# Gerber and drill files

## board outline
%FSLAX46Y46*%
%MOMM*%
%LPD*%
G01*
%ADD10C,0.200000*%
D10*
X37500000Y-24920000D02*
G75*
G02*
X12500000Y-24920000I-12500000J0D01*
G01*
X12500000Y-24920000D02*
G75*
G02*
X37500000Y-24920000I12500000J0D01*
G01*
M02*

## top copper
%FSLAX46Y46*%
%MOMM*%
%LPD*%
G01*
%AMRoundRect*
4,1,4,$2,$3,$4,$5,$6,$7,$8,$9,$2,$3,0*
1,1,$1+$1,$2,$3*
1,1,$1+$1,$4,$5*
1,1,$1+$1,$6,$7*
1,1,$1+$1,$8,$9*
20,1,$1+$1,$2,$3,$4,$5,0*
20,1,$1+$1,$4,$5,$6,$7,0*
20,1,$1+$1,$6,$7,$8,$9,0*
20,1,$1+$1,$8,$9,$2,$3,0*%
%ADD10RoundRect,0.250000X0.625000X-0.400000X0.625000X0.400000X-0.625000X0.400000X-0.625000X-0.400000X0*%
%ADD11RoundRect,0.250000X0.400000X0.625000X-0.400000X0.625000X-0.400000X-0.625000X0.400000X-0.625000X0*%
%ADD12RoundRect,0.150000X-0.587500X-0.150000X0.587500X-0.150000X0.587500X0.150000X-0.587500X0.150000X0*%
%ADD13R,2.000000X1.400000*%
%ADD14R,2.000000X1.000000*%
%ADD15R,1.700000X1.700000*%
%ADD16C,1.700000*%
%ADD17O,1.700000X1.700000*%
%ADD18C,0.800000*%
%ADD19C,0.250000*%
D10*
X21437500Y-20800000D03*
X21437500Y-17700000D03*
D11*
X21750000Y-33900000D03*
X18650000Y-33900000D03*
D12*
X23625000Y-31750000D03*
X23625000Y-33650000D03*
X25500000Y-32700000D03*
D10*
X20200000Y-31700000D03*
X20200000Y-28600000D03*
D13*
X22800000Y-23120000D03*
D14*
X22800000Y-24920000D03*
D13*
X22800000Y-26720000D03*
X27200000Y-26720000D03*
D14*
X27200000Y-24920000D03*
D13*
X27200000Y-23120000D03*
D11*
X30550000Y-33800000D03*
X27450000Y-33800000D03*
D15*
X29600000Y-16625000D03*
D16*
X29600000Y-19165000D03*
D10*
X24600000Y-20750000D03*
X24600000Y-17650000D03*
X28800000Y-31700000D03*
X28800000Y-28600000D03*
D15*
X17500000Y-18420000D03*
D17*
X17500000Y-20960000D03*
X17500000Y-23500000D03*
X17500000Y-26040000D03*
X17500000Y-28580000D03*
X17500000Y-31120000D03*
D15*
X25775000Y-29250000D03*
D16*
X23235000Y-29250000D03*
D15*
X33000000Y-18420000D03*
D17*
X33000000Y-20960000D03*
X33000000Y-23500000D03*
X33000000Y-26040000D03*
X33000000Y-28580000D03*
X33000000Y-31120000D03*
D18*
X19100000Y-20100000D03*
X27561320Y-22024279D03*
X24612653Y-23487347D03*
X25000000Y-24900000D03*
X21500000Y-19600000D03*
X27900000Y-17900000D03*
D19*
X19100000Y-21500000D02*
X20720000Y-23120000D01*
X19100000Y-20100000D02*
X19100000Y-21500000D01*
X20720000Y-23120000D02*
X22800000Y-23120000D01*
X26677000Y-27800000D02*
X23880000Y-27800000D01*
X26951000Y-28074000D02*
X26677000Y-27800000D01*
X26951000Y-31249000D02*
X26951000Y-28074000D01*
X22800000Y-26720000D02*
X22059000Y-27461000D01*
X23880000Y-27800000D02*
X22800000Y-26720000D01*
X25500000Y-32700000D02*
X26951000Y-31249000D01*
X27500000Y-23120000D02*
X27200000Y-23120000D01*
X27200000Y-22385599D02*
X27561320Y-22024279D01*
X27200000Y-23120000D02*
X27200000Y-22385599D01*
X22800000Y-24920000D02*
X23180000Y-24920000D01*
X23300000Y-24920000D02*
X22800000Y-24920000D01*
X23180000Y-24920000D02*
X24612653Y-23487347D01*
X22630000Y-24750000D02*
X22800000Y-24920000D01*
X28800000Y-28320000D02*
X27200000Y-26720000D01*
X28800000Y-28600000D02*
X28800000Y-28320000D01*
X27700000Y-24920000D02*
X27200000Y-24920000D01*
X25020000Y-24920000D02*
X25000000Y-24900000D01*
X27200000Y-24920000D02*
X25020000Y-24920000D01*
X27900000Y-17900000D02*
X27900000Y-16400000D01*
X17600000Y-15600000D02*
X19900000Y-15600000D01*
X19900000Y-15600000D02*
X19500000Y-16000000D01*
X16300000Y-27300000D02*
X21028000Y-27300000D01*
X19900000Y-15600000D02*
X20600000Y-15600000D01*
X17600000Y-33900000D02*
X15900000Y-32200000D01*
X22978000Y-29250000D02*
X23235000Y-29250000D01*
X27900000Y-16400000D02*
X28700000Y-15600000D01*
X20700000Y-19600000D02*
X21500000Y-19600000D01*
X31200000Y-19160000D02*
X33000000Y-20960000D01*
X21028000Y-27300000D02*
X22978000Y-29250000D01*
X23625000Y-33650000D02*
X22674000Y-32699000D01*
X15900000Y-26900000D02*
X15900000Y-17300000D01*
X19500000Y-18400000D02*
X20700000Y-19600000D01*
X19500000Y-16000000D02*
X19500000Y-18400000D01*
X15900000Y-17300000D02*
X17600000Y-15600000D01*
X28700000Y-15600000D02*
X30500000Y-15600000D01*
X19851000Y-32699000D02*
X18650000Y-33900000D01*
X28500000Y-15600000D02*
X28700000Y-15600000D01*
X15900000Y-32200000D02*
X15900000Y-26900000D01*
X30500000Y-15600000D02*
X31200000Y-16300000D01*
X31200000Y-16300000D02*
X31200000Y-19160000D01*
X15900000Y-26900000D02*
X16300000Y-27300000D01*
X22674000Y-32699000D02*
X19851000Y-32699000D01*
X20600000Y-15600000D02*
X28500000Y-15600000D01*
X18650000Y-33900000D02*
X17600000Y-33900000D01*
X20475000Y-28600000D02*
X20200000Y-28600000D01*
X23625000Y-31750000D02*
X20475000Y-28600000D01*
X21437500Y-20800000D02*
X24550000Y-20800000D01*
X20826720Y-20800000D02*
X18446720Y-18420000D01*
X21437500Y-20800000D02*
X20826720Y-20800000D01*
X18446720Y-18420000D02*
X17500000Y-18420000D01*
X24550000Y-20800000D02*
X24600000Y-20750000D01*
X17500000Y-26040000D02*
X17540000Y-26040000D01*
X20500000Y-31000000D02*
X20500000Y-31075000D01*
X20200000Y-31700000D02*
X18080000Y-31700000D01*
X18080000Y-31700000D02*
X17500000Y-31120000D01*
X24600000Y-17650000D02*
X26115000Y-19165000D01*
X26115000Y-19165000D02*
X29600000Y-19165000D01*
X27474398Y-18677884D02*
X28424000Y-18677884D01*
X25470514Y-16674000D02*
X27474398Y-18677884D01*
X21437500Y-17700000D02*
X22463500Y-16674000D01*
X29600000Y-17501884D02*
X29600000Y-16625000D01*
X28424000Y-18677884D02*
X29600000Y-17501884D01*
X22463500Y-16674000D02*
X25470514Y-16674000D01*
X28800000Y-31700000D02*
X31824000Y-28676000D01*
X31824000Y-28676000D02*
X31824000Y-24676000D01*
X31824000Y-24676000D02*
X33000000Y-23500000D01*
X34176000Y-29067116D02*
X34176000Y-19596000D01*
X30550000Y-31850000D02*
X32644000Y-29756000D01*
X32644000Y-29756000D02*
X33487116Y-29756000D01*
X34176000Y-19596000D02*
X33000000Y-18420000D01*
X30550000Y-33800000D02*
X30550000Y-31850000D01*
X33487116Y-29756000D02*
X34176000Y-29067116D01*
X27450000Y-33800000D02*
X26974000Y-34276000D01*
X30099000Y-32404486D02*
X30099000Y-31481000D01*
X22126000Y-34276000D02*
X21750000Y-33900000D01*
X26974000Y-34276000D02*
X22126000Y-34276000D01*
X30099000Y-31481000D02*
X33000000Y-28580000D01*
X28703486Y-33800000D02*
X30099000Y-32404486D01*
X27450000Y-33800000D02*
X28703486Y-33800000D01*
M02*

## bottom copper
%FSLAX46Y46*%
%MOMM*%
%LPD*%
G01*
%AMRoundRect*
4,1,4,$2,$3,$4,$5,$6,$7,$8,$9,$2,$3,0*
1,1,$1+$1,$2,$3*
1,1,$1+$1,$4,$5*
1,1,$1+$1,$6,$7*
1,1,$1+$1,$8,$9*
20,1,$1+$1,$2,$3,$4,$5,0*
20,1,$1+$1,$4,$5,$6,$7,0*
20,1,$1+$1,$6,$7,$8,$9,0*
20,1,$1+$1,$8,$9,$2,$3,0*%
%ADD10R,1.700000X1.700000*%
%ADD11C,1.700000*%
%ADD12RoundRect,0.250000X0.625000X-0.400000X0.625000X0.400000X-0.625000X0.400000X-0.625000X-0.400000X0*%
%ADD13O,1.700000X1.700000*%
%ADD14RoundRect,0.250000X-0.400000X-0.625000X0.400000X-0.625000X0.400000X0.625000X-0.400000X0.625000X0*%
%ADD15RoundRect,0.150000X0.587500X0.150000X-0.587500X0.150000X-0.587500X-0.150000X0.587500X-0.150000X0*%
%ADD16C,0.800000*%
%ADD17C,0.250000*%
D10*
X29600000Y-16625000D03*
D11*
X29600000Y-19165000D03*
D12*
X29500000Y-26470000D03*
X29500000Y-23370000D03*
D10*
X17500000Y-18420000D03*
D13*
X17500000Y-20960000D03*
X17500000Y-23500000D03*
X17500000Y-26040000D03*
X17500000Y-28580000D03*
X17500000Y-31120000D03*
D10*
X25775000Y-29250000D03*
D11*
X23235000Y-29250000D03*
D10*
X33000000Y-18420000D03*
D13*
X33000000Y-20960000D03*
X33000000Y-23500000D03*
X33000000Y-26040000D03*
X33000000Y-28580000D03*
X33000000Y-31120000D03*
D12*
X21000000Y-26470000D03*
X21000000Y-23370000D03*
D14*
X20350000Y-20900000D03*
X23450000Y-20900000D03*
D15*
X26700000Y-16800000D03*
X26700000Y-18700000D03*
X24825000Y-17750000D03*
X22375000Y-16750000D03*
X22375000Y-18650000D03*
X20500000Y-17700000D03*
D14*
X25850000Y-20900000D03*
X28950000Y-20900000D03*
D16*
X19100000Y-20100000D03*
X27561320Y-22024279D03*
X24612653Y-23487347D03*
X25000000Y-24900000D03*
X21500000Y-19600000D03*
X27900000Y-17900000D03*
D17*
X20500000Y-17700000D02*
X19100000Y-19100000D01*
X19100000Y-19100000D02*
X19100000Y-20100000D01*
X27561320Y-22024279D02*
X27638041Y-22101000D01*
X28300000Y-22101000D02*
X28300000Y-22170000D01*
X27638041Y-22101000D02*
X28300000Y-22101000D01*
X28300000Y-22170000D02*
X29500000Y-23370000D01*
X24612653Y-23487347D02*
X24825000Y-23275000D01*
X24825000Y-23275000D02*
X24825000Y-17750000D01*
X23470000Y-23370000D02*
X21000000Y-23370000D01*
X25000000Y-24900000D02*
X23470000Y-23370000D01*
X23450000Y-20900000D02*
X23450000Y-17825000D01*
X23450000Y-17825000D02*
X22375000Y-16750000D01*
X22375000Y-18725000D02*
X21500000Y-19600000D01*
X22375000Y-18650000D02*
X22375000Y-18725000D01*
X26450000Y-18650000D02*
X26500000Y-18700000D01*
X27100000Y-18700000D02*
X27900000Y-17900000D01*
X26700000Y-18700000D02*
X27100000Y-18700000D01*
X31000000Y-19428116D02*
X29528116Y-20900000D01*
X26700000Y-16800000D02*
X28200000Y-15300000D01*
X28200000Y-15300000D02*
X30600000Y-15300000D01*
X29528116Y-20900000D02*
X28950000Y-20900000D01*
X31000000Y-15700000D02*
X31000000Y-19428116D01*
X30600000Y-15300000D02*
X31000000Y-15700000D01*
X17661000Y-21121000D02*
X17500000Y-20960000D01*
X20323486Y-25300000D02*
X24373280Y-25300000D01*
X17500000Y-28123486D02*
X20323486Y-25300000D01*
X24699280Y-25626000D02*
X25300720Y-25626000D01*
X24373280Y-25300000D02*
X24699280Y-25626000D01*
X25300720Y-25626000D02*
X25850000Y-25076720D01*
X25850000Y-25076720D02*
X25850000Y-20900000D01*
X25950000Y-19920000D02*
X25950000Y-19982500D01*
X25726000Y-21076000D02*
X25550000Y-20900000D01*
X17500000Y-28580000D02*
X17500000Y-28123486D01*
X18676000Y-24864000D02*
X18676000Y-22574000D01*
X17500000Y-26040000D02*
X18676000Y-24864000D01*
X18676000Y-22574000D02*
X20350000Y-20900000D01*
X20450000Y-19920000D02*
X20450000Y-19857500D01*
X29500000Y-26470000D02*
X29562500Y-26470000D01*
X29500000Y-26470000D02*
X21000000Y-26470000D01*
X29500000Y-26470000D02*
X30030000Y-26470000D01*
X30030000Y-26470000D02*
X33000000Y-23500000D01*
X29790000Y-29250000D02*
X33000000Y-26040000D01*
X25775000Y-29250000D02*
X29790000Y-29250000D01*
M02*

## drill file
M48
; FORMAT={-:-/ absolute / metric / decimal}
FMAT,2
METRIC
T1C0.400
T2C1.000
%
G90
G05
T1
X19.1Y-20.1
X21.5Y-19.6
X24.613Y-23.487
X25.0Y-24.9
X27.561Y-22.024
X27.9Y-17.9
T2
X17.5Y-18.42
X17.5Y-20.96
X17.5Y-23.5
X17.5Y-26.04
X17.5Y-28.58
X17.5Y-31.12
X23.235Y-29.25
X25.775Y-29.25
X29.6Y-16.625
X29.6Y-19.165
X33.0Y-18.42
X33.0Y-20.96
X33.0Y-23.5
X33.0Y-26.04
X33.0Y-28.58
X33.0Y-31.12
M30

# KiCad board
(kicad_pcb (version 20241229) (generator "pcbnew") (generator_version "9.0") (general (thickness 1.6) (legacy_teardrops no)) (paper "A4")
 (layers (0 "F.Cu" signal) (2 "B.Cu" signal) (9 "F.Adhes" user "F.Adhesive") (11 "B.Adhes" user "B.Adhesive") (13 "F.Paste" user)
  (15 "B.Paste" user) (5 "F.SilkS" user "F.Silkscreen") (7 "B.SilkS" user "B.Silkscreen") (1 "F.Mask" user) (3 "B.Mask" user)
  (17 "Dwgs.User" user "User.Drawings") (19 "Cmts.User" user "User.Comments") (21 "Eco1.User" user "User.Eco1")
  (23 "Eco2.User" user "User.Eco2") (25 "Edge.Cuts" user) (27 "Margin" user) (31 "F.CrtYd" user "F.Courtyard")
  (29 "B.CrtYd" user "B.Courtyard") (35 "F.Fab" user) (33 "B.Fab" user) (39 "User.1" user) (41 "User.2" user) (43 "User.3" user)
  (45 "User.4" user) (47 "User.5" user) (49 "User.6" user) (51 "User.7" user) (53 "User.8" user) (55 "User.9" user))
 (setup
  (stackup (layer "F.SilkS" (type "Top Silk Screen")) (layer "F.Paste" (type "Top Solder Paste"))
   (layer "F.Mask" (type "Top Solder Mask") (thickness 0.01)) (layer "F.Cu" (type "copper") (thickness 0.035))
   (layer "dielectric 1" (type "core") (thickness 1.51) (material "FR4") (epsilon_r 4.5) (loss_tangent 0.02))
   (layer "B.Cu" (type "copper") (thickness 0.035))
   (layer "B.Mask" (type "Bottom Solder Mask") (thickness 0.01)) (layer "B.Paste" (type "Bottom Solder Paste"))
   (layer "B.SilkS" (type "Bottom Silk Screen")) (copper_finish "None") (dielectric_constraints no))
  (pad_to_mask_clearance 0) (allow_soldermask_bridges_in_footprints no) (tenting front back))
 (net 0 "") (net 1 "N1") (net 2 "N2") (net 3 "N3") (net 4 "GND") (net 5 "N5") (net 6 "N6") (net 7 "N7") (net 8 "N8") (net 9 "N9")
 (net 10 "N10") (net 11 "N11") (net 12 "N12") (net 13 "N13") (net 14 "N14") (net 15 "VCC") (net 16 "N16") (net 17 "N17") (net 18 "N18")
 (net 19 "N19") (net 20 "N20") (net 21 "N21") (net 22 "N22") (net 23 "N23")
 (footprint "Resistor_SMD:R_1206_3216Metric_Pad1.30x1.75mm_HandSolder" (layer "F.Cu") (at 21.4375 19.25 90)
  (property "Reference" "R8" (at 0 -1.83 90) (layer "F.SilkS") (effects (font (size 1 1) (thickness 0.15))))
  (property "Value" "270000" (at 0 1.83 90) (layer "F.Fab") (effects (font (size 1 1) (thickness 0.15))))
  (pad "1" smd roundrect (at -1.55 0 90) (size 1.3 1.75) (layers "F.Cu" "F.Mask" "F.Paste") (roundrect_rratio 0.192308) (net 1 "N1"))
  (pad "2" smd roundrect (at 1.55 0 90) (size 1.3 1.75) (layers "F.Cu" "F.Mask" "F.Paste") (roundrect_rratio 0.192308) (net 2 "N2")))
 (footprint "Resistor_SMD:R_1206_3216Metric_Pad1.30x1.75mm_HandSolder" (layer "F.Cu") (at 20.2 33.9 180)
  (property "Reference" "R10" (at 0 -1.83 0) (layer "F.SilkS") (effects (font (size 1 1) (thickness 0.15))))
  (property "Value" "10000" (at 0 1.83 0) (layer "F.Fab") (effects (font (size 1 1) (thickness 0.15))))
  (pad "1" smd roundrect (at -1.55 0 180) (size 1.3 1.75) (layers "F.Cu" "F.Mask" "F.Paste") (roundrect_rratio 0.192308) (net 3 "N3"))
  (pad "2" smd roundrect (at 1.55 0 180) (size 1.3 1.75) (layers "F.Cu" "F.Mask" "F.Paste") (roundrect_rratio 0.192308) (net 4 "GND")))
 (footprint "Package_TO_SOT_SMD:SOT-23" (layer "F.Cu") (at 24.5625 32.7)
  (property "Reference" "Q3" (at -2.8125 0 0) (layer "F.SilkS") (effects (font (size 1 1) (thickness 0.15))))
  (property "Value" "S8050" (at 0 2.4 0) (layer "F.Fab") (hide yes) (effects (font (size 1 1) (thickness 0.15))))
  (pad "1" smd roundrect (at -0.9375 -0.95) (size 1.475 0.6) (layers "F.Cu" "F.Mask" "F.Paste") (roundrect_rratio 0.25) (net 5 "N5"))
  (pad "2" smd roundrect (at -0.9375 0.95) (size 1.475 0.6) (layers "F.Cu" "F.Mask" "F.Paste") (roundrect_rratio 0.25) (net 4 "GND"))
  (pad "3" smd roundrect (at 0.9375 0) (size 1.475 0.6) (layers "F.Cu" "F.Mask" "F.Paste") (roundrect_rratio 0.25) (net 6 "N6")))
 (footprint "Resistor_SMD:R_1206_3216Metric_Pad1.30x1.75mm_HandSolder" (layer "F.Cu") (at 20.2 30.15 90)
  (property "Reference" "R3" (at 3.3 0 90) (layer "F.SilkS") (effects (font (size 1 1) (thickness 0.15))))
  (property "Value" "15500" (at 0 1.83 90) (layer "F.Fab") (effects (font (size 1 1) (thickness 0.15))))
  (pad "1" smd roundrect (at -1.55 0 90) (size 1.3 1.75) (layers "F.Cu" "F.Mask" "F.Paste") (roundrect_rratio 0.192308) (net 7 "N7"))
  (pad "2" smd roundrect (at 1.55 0 90) (size 1.3 1.75) (layers "F.Cu" "F.Mask" "F.Paste") (roundrect_rratio 0.192308) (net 5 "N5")))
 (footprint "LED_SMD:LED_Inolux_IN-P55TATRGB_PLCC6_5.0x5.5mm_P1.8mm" (layer "F.Cu") (at 25 24.92)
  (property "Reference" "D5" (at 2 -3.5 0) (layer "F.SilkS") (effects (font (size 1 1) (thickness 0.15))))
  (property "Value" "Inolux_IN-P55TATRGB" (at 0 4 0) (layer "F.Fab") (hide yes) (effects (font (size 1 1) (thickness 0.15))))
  (pad "1" smd rect (at -2.2 -1.8) (size 2 1.4) (layers "F.Cu" "F.Mask" "F.Paste") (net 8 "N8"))
  (pad "2" smd rect (at -2.2 0) (size 2 1) (layers "F.Cu" "F.Mask" "F.Paste") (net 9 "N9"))
  (pad "3" smd rect (at -2.2 1.8) (size 2 1.4) (layers "F.Cu" "F.Mask" "F.Paste") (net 6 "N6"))
  (pad "4" smd rect (at 2.2 1.8) (size 2 1.4) (layers "F.Cu" "F.Mask" "F.Paste") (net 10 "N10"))
  (pad "5" smd rect (at 2.2 0) (size 2 1) (layers "F.Cu" "F.Mask" "F.Paste") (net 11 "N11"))
  (pad "6" smd rect (at 2.2 -1.8) (size 2 1.4) (layers "F.Cu" "F.Mask" "F.Paste") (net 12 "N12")))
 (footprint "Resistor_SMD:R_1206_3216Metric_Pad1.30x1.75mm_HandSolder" (layer "F.Cu") (at 29 33.8 180)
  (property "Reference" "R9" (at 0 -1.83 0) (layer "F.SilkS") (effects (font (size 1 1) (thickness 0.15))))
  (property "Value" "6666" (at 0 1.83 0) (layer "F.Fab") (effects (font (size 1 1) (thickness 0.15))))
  (pad "1" smd roundrect (at -1.55 0 180) (size 1.3 1.75) (layers "F.Cu" "F.Mask" "F.Paste") (roundrect_rratio 0.192308) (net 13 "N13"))
  (pad "2" smd roundrect (at 1.55 0 180) (size 1.3 1.75) (layers "F.Cu" "F.Mask" "F.Paste") (roundrect_rratio 0.192308) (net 3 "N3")))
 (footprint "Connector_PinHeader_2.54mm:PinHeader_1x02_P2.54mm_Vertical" (layer "F.Cu") (at 29.6 16.625)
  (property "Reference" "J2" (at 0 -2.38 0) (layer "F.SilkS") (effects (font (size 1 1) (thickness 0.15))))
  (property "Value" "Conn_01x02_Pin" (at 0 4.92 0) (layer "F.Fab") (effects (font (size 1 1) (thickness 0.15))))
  (pad "1" thru_hole rect (at 0 0) (size 1.7 1.7) (drill 1) (layers "*.Cu" "*.Mask") (remove_unused_layers no) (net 2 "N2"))
  (pad "2" thru_hole circle (at 0 2.54) (size 1.7 1.7) (drill 1) (layers "*.Cu" "*.Mask") (remove_unused_layers no) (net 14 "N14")))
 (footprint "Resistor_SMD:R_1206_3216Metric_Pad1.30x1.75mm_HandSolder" (layer "F.Cu") (at 24.6 19.2 90)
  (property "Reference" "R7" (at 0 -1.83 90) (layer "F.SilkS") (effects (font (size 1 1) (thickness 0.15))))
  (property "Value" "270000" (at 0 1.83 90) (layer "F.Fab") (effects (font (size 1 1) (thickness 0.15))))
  (pad "1" smd roundrect (at -1.55 0 90) (size 1.3 1.75) (layers "F.Cu" "F.Mask" "F.Paste") (roundrect_rratio 0.192308) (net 1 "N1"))
  (pad "2" smd roundrect (at 1.55 0 90) (size 1.3 1.75) (layers "F.Cu" "F.Mask" "F.Paste") (roundrect_rratio 0.192308) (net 14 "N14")))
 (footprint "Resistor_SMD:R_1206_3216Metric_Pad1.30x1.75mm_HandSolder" (layer "F.Cu") (at 28.8 30.15 90)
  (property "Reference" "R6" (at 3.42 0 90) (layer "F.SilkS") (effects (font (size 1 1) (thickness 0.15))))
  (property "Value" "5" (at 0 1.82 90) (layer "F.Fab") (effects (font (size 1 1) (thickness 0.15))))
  (pad "1" smd roundrect (at -1.55 0 90) (size 1.3 1.75) (layers "F.Cu" "F.Mask" "F.Paste") (roundrect_rratio 0.192308) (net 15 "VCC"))
  (pad "2" smd roundrect (at 1.55 0 90) (size 1.3 1.75) (layers "F.Cu" "F.Mask" "F.Paste") (roundrect_rratio 0.192308) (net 10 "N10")))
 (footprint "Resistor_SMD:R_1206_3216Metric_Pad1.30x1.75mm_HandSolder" (layer "B.Cu") (at 29.5 24.92 90)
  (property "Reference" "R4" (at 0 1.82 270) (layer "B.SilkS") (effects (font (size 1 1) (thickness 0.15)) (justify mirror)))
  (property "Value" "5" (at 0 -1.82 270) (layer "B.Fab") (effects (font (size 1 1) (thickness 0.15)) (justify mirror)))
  (pad "1" smd roundrect (at -1.55 0 90) (size 1.3 1.75) (layers "B.Cu" "B.Mask" "B.Paste") (roundrect_rratio 0.192308) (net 15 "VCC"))
  (pad "2" smd roundrect (at 1.55 0 90) (size 1.3 1.75) (layers "B.Cu" "B.Mask" "B.Paste") (roundrect_rratio 0.192308) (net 12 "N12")))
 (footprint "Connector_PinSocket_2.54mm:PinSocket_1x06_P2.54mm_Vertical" (layer "B.Cu") (at 17.5 18.42 180)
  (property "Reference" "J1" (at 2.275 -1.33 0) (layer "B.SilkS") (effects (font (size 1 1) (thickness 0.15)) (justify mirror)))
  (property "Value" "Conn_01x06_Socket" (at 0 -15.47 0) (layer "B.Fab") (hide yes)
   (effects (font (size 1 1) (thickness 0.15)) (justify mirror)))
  (pad "1" thru_hole rect (at 0 0 180) (size 1.7 1.7) (drill 1) (layers "*.Cu" "*.Mask") (remove_unused_layers no) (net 1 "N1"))
  (pad "2" thru_hole oval (at 0 -2.54 180) (size 1.7 1.7) (drill 1) (layers "*.Cu" "*.Mask") (remove_unused_layers no) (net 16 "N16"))
  (pad "3" thru_hole oval (at 0 -5.08 180) (size 1.7 1.7) (drill 1) (layers "*.Cu" "*.Mask") (remove_unused_layers no) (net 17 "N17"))
  (pad "4" thru_hole oval (at 0 -7.62 180) (size 1.7 1.7) (drill 1) (layers "*.Cu" "*.Mask") (remove_unused_layers no) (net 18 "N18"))
  (pad "5" thru_hole oval (at 0 -10.16 180) (size 1.7 1.7) (drill 1) (layers "*.Cu" "*.Mask") (remove_unused_layers no) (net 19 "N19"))
  (pad "6" thru_hole oval (at 0 -12.7 180) (size 1.7 1.7) (drill 1) (layers "*.Cu" "*.Mask") (remove_unused_layers no) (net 7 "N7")))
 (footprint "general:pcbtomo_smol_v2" (layer "B.Cu") (at 24.275 29.5 180)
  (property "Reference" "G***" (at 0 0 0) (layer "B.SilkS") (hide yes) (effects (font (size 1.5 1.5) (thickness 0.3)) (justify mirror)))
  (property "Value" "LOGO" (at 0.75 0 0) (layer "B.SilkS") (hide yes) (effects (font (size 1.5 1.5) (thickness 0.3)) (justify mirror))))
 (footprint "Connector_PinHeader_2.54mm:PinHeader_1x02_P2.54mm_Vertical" (layer "B.Cu") (at 25.775 29.25 90)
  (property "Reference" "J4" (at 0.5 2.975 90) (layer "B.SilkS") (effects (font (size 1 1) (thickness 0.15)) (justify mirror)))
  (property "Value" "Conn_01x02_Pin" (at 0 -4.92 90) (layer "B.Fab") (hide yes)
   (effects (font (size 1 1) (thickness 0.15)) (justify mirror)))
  (pad "1" thru_hole rect (at 0 0 90) (size 1.7 1.7) (drill 1) (layers "*.Cu" "*.Mask") (remove_unused_layers no) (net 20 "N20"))
  (pad "2" thru_hole circle (at 0 -2.54 90) (size 1.7 1.7) (drill 1) (layers "*.Cu" "*.Mask") (remove_unused_layers no) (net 4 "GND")))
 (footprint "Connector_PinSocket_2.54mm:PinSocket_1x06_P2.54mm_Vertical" (layer "B.Cu") (at 33 18.42 180)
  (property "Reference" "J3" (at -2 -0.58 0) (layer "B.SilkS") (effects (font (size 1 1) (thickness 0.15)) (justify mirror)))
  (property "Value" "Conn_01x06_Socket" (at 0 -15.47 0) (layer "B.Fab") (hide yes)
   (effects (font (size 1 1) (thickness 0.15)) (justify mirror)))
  (pad "1" thru_hole rect (at 0 0 180) (size 1.7 1.7) (drill 1) (layers "*.Cu" "*.Mask") (remove_unused_layers no) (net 13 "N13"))
  (pad "2" thru_hole oval (at 0 -2.54 180) (size 1.7 1.7) (drill 1) (layers "*.Cu" "*.Mask") (remove_unused_layers no) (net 4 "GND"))
  (pad "3" thru_hole oval (at 0 -5.08 180) (size 1.7 1.7) (drill 1) (layers "*.Cu" "*.Mask") (remove_unused_layers no) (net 15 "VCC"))
  (pad "4" thru_hole oval (at 0 -7.62 180) (size 1.7 1.7) (drill 1) (layers "*.Cu" "*.Mask") (remove_unused_layers no) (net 20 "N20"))
  (pad "5" thru_hole oval (at 0 -10.16 180) (size 1.7 1.7) (drill 1) (layers "*.Cu" "*.Mask") (remove_unused_layers no) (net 3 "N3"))
  (pad "6" thru_hole oval (at 0 -12.7 180) (size 1.7 1.7) (drill 1) (layers "*.Cu" "*.Mask") (remove_unused_layers no) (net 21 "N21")))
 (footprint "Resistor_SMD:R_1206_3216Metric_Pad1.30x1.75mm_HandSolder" (layer "B.Cu") (at 21 24.92 90)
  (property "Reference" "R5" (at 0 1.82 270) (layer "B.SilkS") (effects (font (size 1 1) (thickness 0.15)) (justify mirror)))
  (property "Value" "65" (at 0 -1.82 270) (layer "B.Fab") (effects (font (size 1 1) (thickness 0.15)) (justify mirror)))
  (pad "1" smd roundrect (at -1.55 0 90) (size 1.3 1.75) (layers "B.Cu" "B.Mask" "B.Paste") (roundrect_rratio 0.192308) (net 15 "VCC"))
  (pad "2" smd roundrect (at 1.55 0 90) (size 1.3 1.75) (layers "B.Cu" "B.Mask" "B.Paste") (roundrect_rratio 0.192308) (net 11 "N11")))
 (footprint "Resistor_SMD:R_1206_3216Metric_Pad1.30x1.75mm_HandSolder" (layer "B.Cu") (at 21.9 20.9)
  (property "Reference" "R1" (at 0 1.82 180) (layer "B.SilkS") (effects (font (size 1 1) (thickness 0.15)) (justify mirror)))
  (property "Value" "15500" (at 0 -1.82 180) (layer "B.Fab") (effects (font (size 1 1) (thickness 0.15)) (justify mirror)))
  (pad "1" smd roundrect (at -1.55 0) (size 1.3 1.75) (layers "B.Cu" "B.Mask" "B.Paste") (roundrect_rratio 0.192308) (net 18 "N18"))
  (pad "2" smd roundrect (at 1.55 0) (size 1.3 1.75) (layers "B.Cu" "B.Mask" "B.Paste") (roundrect_rratio 0.192308) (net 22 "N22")))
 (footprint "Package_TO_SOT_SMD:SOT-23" (layer "B.Cu") (at 25.7625 17.75 180)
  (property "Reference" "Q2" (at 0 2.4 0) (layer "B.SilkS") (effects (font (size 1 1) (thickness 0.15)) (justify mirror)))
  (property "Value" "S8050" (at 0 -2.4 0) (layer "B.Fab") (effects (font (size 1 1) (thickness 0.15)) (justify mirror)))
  (pad "1" smd roundrect (at -0.9375 0.95 180) (size 1.475 0.6) (layers "B.Cu" "B.Mask" "B.Paste") (roundrect_rratio 0.25) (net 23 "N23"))
  (pad "2" smd roundrect (at -0.9375 -0.95 180) (size 1.475 0.6) (layers "B.Cu" "B.Mask" "B.Paste") (roundrect_rratio 0.25) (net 4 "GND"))
  (pad "3" smd roundrect (at 0.9375 0 180) (size 1.475 0.6) (layers "B.Cu" "B.Mask" "B.Paste") (roundrect_rratio 0.25) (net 9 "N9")))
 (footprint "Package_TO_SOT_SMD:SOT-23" (layer "B.Cu") (at 21.4375 17.7 180)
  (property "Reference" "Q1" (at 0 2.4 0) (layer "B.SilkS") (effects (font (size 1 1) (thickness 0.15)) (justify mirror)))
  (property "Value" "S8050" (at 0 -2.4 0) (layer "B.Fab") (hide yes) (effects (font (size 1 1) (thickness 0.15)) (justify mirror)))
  (pad "1" smd roundrect (at -0.9375 0.95 180) (size 1.475 0.6) (layers "B.Cu" "B.Mask" "B.Paste") (roundrect_rratio 0.25) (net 22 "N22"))
  (pad "2" smd roundrect (at -0.9375 -0.95 180) (size 1.475 0.6) (layers "B.Cu" "B.Mask" "B.Paste") (roundrect_rratio 0.25) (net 4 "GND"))
  (pad "3" smd roundrect (at 0.9375 0 180) (size 1.475 0.6) (layers "B.Cu" "B.Mask" "B.Paste") (roundrect_rratio 0.25) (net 8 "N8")))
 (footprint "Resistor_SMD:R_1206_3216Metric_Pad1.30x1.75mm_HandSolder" (layer "B.Cu") (at 27.4 20.9)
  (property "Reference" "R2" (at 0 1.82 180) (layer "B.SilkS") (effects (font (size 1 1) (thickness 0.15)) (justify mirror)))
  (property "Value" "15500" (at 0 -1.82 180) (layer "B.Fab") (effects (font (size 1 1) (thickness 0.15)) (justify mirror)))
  (pad "1" smd roundrect (at -1.55 0) (size 1.3 1.75) (layers "B.Cu" "B.Mask" "B.Paste") (roundrect_rratio 0.192308) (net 19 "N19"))
  (pad "2" smd roundrect (at 1.55 0) (size 1.3 1.75) (layers "B.Cu" "B.Mask" "B.Paste") (roundrect_rratio 0.192308) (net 23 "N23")))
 (gr_circle (center 25 24.92) (end 37.5 24.92) (stroke (width 0.2) (type default)) (fill no) (layer "Edge.Cuts"))
 (segment (start 19.1 21.5) (end 20.72 23.12) (width 0.25) (layer "F.Cu") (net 8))
 (segment (start 19.1 20.1) (end 19.1 21.5) (width 0.25) (layer "F.Cu") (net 8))
 (segment (start 20.72 23.12) (end 22.8 23.12) (width 0.25) (layer "F.Cu") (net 8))
 (via (at 19.1 20.1) (size 0.8) (drill 0.4) (layers "F.Cu" "B.Cu") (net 8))
 (segment (start 20.5 17.7) (end 19.1 19.1) (width 0.25) (layer "B.Cu") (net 8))
 (segment (start 19.1 19.1) (end 19.1 20.1) (width 0.25) (layer "B.Cu") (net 8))
 (segment (start 26.677 27.8) (end 23.88 27.8) (width 0.25) (layer "F.Cu") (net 6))
 (segment (start 26.951 28.074) (end 26.677 27.8) (width 0.25) (layer "F.Cu") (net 6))
 (segment (start 26.951 31.249) (end 26.951 28.074) (width 0.25) (layer "F.Cu") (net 6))
 (segment (start 22.8 26.72) (end 22.059 27.461) (width 0.25) (layer "F.Cu") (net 6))
 (segment (start 23.88 27.8) (end 22.8 26.72) (width 0.25) (layer "F.Cu") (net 6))
 (segment (start 25.5 32.7) (end 26.951 31.249) (width 0.25) (layer "F.Cu") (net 6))
 (segment (start 27.5 23.12) (end 27.2 23.12) (width 0.25) (layer "F.Cu") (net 12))
 (segment (start 27.2 22.385599) (end 27.56132 22.024279) (width 0.25) (layer "F.Cu") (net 12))
 (segment (start 27.2 23.12) (end 27.2 22.385599) (width 0.25) (layer "F.Cu") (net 12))
 (via (at 27.56132 22.024279) (size 0.8) (drill 0.4) (layers "F.Cu" "B.Cu") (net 12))
 (segment (start 27.56132 22.024279) (end 27.638041 22.101) (width 0.25) (layer "B.Cu") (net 12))
 (segment (start 28.3 22.101) (end 28.3 22.17) (width 0.25) (layer "B.Cu") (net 12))
 (segment (start 27.638041 22.101) (end 28.3 22.101) (width 0.25) (layer "B.Cu") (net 12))
 (segment (start 28.3 22.17) (end 29.5 23.37) (width 0.25) (layer "B.Cu") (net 12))
 (segment (start 22.8 24.92) (end 23.18 24.92) (width 0.25) (layer "F.Cu") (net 9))
 (segment (start 23.3 24.92) (end 22.8 24.92) (width 0.25) (layer "F.Cu") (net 9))
 (segment (start 23.18 24.92) (end 24.612653 23.487347) (width 0.25) (layer "F.Cu") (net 9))
 (segment (start 22.63 24.75) (end 22.8 24.92) (width 0.25) (layer "F.Cu") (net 9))
 (via (at 24.612653 23.487347) (size 0.8) (drill 0.4) (layers "F.Cu" "B.Cu") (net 9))
 (segment (start 24.612653 23.487347) (end 24.825 23.275) (width 0.25) (layer "B.Cu") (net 9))
 (segment (start 24.825 23.275) (end 24.825 17.75) (width 0.25) (layer "B.Cu") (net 9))
 (segment (start 28.8 28.32) (end 27.2 26.72) (width 0.25) (layer "F.Cu") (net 10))
 (segment (start 28.8 28.6) (end 28.8 28.32) (width 0.25) (layer "F.Cu") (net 10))
 (segment (start 27.7 24.92) (end 27.2 24.92) (width 0.25) (layer "F.Cu") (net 11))
 (segment (start 25.02 24.92) (end 25 24.9) (width 0.25) (layer "F.Cu") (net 11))
 (segment (start 27.2 24.92) (end 25.02 24.92) (width 0.25) (layer "F.Cu") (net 11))
 (via (at 25 24.9) (size 0.8) (drill 0.4) (layers "F.Cu" "B.Cu") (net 11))
 (segment (start 23.47 23.37) (end 21 23.37) (width 0.25) (layer "B.Cu") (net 11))
 (segment (start 25 24.9) (end 23.47 23.37) (width 0.25) (layer "B.Cu") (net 11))
 (segment (start 23.45 20.9) (end 23.45 17.825) (width 0.25) (layer "B.Cu") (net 22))
 (segment (start 23.45 17.825) (end 22.375 16.75) (width 0.25) (layer "B.Cu") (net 22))
 (segment (start 27.9 17.9) (end 27.9 16.4) (width 0.25) (layer "F.Cu") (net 4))
 (segment (start 17.6 15.6) (end 19.9 15.6) (width 0.25) (layer "F.Cu") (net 4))
 (segment (start 19.9 15.6) (end 19.5 16) (width 0.25) (layer "F.Cu") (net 4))
 (segment (start 16.3 27.3) (end 21.028 27.3) (width 0.25) (layer "F.Cu") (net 4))
 (segment (start 19.9 15.6) (end 20.6 15.6) (width 0.25) (layer "F.Cu") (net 4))
 (segment (start 17.6 33.9) (end 15.9 32.2) (width 0.25) (layer "F.Cu") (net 4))
 (segment (start 22.978 29.25) (end 23.235 29.25) (width 0.25) (layer "F.Cu") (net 4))
 (segment (start 27.9 16.4) (end 28.7 15.6) (width 0.25) (layer "F.Cu") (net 4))
 (segment (start 20.7 19.6) (end 21.5 19.6) (width 0.25) (layer "F.Cu") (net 4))
 (segment (start 31.2 19.16) (end 33 20.96) (width 0.25) (layer "F.Cu") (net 4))
 (segment (start 21.028 27.3) (end 22.978 29.25) (width 0.25) (layer "F.Cu") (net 4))
 (segment (start 23.625 33.65) (end 22.674 32.699) (width 0.25) (layer "F.Cu") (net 4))
 (segment (start 15.9 26.9) (end 15.9 17.3) (width 0.25) (layer "F.Cu") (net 4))
 (segment (start 19.5 18.4) (end 20.7 19.6) (width 0.25) (layer "F.Cu") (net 4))
 (segment (start 19.5 16) (end 19.5 18.4) (width 0.25) (layer "F.Cu") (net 4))
 (segment (start 15.9 17.3) (end 17.6 15.6) (width 0.25) (layer "F.Cu") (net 4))
 (segment (start 28.7 15.6) (end 30.5 15.6) (width 0.25) (layer "F.Cu") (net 4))
 (segment (start 19.851 32.699) (end 18.65 33.9) (width 0.25) (layer "F.Cu") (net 4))
 (segment (start 28.5 15.6) (end 28.7 15.6) (width 0.25) (layer "F.Cu") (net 4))
 (segment (start 15.9 32.2) (end 15.9 26.9) (width 0.25) (layer "F.Cu") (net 4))
 (segment (start 30.5 15.6) (end 31.2 16.3) (width 0.25) (layer "F.Cu") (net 4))
 (segment (start 31.2 16.3) (end 31.2 19.16) (width 0.25) (layer "F.Cu") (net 4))
 (segment (start 15.9 26.9) (end 16.3 27.3) (width 0.25) (layer "F.Cu") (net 4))
 (segment (start 22.674 32.699) (end 19.851 32.699) (width 0.25) (layer "F.Cu") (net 4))
 (segment (start 20.6 15.6) (end 28.5 15.6) (width 0.25) (layer "F.Cu") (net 4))
 (segment (start 18.65 33.9) (end 17.6 33.9) (width 0.25) (layer "F.Cu") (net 4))
 (via (at 21.5 19.6) (size 0.8) (drill 0.4) (layers "F.Cu" "B.Cu") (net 4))
 (via (at 27.9 17.9) (size 0.8) (drill 0.4) (layers "F.Cu" "B.Cu") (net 4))
 (segment (start 22.375 18.725) (end 21.5 19.6) (width 0.25) (layer "B.Cu") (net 4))
 (segment (start 22.375 18.65) (end 22.375 18.725) (width 0.25) (layer "B.Cu") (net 4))
 (segment (start 26.45 18.65) (end 26.5 18.7) (width 0.25) (layer "B.Cu") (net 4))
 (segment (start 27.1 18.7) (end 27.9 17.9) (width 0.25) (layer "B.Cu") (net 4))
 (segment (start 26.7 18.7) (end 27.1 18.7) (width 0.25) (layer "B.Cu") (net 4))
 (segment (start 31 19.428116) (end 29.528116 20.9) (width 0.25) (layer "B.Cu") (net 23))
 (segment (start 26.7 16.8) (end 28.2 15.3) (width 0.25) (layer "B.Cu") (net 23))
 (segment (start 28.2 15.3) (end 30.6 15.3) (width 0.25) (layer "B.Cu") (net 23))
 (segment (start 29.528116 20.9) (end 28.95 20.9) (width 0.25) (layer "B.Cu") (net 23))
 (segment (start 31 15.7) (end 31 19.428116) (width 0.25) (layer "B.Cu") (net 23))
 (segment (start 30.6 15.3) (end 31 15.7) (width 0.25) (layer "B.Cu") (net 23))
 (segment (start 20.475 28.6) (end 20.2 28.6) (width 0.25) (layer "F.Cu") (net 5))
 (segment (start 23.625 31.75) (end 20.475 28.6) (width 0.25) (layer "F.Cu") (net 5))
 (segment (start 17.661 21.121) (end 17.5 20.96) (width 0.25) (layer "B.Cu") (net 16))
 (segment (start 20.323486 25.3) (end 24.37328 25.3) (width 0.25) (layer "B.Cu") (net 19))
 (segment (start 17.5 28.123486) (end 20.323486 25.3) (width 0.25) (layer "B.Cu") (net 19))
 (segment (start 24.69928 25.626) (end 25.30072 25.626) (width 0.25) (layer "B.Cu") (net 19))
 (segment (start 24.37328 25.3) (end 24.69928 25.626) (width 0.25) (layer "B.Cu") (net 19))
 (segment (start 25.30072 25.626) (end 25.85 25.07672) (width 0.25) (layer "B.Cu") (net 19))
 (segment (start 25.85 25.07672) (end 25.85 20.9) (width 0.25) (layer "B.Cu") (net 19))
 (segment (start 25.95 19.92) (end 25.95 19.9825) (width 0.25) (layer "B.Cu") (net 19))
 (segment (start 25.726 21.076) (end 25.55 20.9) (width 0.25) (layer "B.Cu") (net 19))
 (segment (start 17.5 28.58) (end 17.5 28.123486) (width 0.25) (layer "B.Cu") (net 19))
 (segment (start 21.4375 20.8) (end 24.55 20.8) (width 0.25) (layer "F.Cu") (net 1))
 (segment (start 20.82672 20.8) (end 18.44672 18.42) (width 0.25) (layer "F.Cu") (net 1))
 (segment (start 21.4375 20.8) (end 20.82672 20.8) (width 0.25) (layer "F.Cu") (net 1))
 (segment (start 18.44672 18.42) (end 17.5 18.42) (width 0.25) (layer "F.Cu") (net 1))
 (segment (start 24.55 20.8) (end 24.6 20.75) (width 0.25) (layer "F.Cu") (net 1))
 (segment (start 17.5 26.04) (end 17.54 26.04) (width 0.25) (layer "F.Cu") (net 18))
 (segment (start 18.676 24.864) (end 18.676 22.574) (width 0.25) (layer "B.Cu") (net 18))
 (segment (start 17.5 26.04) (end 18.676 24.864) (width 0.25) (layer "B.Cu") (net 18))
 (segment (start 18.676 22.574) (end 20.35 20.9) (width 0.25) (layer "B.Cu") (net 18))
 (segment (start 20.45 19.92) (end 20.45 19.8575) (width 0.25) (layer "B.Cu") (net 18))
 (segment (start 20.5 31) (end 20.5 31.075) (width 0.25) (layer "F.Cu") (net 7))
 (segment (start 20.2 31.7) (end 18.08 31.7) (width 0.25) (layer "F.Cu") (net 7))
 (segment (start 18.08 31.7) (end 17.5 31.12) (width 0.25) (layer "F.Cu") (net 7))
 (segment (start 24.6 17.65) (end 26.115 19.165) (width 0.25) (layer "F.Cu") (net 14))
 (segment (start 26.115 19.165) (end 29.6 19.165) (width 0.25) (layer "F.Cu") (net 14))
 (segment (start 27.474398 18.677884) (end 28.424 18.677884) (width 0.25) (layer "F.Cu") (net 2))
 (segment (start 25.470514 16.674) (end 27.474398 18.677884) (width 0.25) (layer "F.Cu") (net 2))
 (segment (start 21.4375 17.7) (end 22.4635 16.674) (width 0.25) (layer "F.Cu") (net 2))
 (segment (start 29.6 17.501884) (end 29.6 16.625) (width 0.25) (layer "F.Cu") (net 2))
 (segment (start 28.424 18.677884) (end 29.6 17.501884) (width 0.25) (layer "F.Cu") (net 2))
 (segment (start 22.4635 16.674) (end 25.470514 16.674) (width 0.25) (layer "F.Cu") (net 2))
 (segment (start 28.8 31.7) (end 31.824 28.676) (width 0.25) (layer "F.Cu") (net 15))
 (segment (start 31.824 28.676) (end 31.824 24.676) (width 0.25) (layer "F.Cu") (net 15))
 (segment (start 31.824 24.676) (end 33 23.5) (width 0.25) (layer "F.Cu") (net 15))
 (segment (start 29.5 26.47) (end 29.5625 26.47) (width 0.25) (layer "B.Cu") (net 15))
 (segment (start 29.5 26.47) (end 21 26.47) (width 0.25) (layer "B.Cu") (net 15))
 (segment (start 29.5 26.47) (end 30.03 26.47) (width 0.25) (layer "B.Cu") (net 15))
 (segment (start 30.03 26.47) (end 33 23.5) (width 0.25) (layer "B.Cu") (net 15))
 (segment (start 29.79 29.25) (end 33 26.04) (width 0.25) (layer "B.Cu") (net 20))
 (segment (start 25.775 29.25) (end 29.79 29.25) (width 0.25) (layer "B.Cu") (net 20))
 (segment (start 34.176 29.067116) (end 34.176 19.596) (width 0.25) (layer "F.Cu") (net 13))
 (segment (start 30.55 31.85) (end 32.644 29.756) (width 0.25) (layer "F.Cu") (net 13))
 (segment (start 32.644 29.756) (end 33.487116 29.756) (width 0.25) (layer "F.Cu") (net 13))
 (segment (start 34.176 19.596) (end 33 18.42) (width 0.25) (layer "F.Cu") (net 13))
 (segment (start 30.55 33.8) (end 30.55 31.85) (width 0.25) (layer "F.Cu") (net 13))
 (segment (start 33.487116 29.756) (end 34.176 29.067116) (width 0.25) (layer "F.Cu") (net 13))
 (segment (start 27.45 33.8) (end 26.974 34.276) (width 0.25) (layer "F.Cu") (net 3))
 (segment (start 30.099 32.404486) (end 30.099 31.481) (width 0.25) (layer "F.Cu") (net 3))
 (segment (start 22.126 34.276) (end 21.75 33.9) (width 0.25) (layer "F.Cu") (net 3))
 (segment (start 26.974 34.276) (end 22.126 34.276) (width 0.25) (layer "F.Cu") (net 3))
 (segment (start 30.099 31.481) (end 33 28.58) (width 0.25) (layer "F.Cu") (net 3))
 (segment (start 28.703486 33.8) (end 30.099 32.404486) (width 0.25) (layer "F.Cu") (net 3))
 (segment (start 27.45 33.8) (end 28.703486 33.8) (width 0.25) (layer "F.Cu") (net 3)))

